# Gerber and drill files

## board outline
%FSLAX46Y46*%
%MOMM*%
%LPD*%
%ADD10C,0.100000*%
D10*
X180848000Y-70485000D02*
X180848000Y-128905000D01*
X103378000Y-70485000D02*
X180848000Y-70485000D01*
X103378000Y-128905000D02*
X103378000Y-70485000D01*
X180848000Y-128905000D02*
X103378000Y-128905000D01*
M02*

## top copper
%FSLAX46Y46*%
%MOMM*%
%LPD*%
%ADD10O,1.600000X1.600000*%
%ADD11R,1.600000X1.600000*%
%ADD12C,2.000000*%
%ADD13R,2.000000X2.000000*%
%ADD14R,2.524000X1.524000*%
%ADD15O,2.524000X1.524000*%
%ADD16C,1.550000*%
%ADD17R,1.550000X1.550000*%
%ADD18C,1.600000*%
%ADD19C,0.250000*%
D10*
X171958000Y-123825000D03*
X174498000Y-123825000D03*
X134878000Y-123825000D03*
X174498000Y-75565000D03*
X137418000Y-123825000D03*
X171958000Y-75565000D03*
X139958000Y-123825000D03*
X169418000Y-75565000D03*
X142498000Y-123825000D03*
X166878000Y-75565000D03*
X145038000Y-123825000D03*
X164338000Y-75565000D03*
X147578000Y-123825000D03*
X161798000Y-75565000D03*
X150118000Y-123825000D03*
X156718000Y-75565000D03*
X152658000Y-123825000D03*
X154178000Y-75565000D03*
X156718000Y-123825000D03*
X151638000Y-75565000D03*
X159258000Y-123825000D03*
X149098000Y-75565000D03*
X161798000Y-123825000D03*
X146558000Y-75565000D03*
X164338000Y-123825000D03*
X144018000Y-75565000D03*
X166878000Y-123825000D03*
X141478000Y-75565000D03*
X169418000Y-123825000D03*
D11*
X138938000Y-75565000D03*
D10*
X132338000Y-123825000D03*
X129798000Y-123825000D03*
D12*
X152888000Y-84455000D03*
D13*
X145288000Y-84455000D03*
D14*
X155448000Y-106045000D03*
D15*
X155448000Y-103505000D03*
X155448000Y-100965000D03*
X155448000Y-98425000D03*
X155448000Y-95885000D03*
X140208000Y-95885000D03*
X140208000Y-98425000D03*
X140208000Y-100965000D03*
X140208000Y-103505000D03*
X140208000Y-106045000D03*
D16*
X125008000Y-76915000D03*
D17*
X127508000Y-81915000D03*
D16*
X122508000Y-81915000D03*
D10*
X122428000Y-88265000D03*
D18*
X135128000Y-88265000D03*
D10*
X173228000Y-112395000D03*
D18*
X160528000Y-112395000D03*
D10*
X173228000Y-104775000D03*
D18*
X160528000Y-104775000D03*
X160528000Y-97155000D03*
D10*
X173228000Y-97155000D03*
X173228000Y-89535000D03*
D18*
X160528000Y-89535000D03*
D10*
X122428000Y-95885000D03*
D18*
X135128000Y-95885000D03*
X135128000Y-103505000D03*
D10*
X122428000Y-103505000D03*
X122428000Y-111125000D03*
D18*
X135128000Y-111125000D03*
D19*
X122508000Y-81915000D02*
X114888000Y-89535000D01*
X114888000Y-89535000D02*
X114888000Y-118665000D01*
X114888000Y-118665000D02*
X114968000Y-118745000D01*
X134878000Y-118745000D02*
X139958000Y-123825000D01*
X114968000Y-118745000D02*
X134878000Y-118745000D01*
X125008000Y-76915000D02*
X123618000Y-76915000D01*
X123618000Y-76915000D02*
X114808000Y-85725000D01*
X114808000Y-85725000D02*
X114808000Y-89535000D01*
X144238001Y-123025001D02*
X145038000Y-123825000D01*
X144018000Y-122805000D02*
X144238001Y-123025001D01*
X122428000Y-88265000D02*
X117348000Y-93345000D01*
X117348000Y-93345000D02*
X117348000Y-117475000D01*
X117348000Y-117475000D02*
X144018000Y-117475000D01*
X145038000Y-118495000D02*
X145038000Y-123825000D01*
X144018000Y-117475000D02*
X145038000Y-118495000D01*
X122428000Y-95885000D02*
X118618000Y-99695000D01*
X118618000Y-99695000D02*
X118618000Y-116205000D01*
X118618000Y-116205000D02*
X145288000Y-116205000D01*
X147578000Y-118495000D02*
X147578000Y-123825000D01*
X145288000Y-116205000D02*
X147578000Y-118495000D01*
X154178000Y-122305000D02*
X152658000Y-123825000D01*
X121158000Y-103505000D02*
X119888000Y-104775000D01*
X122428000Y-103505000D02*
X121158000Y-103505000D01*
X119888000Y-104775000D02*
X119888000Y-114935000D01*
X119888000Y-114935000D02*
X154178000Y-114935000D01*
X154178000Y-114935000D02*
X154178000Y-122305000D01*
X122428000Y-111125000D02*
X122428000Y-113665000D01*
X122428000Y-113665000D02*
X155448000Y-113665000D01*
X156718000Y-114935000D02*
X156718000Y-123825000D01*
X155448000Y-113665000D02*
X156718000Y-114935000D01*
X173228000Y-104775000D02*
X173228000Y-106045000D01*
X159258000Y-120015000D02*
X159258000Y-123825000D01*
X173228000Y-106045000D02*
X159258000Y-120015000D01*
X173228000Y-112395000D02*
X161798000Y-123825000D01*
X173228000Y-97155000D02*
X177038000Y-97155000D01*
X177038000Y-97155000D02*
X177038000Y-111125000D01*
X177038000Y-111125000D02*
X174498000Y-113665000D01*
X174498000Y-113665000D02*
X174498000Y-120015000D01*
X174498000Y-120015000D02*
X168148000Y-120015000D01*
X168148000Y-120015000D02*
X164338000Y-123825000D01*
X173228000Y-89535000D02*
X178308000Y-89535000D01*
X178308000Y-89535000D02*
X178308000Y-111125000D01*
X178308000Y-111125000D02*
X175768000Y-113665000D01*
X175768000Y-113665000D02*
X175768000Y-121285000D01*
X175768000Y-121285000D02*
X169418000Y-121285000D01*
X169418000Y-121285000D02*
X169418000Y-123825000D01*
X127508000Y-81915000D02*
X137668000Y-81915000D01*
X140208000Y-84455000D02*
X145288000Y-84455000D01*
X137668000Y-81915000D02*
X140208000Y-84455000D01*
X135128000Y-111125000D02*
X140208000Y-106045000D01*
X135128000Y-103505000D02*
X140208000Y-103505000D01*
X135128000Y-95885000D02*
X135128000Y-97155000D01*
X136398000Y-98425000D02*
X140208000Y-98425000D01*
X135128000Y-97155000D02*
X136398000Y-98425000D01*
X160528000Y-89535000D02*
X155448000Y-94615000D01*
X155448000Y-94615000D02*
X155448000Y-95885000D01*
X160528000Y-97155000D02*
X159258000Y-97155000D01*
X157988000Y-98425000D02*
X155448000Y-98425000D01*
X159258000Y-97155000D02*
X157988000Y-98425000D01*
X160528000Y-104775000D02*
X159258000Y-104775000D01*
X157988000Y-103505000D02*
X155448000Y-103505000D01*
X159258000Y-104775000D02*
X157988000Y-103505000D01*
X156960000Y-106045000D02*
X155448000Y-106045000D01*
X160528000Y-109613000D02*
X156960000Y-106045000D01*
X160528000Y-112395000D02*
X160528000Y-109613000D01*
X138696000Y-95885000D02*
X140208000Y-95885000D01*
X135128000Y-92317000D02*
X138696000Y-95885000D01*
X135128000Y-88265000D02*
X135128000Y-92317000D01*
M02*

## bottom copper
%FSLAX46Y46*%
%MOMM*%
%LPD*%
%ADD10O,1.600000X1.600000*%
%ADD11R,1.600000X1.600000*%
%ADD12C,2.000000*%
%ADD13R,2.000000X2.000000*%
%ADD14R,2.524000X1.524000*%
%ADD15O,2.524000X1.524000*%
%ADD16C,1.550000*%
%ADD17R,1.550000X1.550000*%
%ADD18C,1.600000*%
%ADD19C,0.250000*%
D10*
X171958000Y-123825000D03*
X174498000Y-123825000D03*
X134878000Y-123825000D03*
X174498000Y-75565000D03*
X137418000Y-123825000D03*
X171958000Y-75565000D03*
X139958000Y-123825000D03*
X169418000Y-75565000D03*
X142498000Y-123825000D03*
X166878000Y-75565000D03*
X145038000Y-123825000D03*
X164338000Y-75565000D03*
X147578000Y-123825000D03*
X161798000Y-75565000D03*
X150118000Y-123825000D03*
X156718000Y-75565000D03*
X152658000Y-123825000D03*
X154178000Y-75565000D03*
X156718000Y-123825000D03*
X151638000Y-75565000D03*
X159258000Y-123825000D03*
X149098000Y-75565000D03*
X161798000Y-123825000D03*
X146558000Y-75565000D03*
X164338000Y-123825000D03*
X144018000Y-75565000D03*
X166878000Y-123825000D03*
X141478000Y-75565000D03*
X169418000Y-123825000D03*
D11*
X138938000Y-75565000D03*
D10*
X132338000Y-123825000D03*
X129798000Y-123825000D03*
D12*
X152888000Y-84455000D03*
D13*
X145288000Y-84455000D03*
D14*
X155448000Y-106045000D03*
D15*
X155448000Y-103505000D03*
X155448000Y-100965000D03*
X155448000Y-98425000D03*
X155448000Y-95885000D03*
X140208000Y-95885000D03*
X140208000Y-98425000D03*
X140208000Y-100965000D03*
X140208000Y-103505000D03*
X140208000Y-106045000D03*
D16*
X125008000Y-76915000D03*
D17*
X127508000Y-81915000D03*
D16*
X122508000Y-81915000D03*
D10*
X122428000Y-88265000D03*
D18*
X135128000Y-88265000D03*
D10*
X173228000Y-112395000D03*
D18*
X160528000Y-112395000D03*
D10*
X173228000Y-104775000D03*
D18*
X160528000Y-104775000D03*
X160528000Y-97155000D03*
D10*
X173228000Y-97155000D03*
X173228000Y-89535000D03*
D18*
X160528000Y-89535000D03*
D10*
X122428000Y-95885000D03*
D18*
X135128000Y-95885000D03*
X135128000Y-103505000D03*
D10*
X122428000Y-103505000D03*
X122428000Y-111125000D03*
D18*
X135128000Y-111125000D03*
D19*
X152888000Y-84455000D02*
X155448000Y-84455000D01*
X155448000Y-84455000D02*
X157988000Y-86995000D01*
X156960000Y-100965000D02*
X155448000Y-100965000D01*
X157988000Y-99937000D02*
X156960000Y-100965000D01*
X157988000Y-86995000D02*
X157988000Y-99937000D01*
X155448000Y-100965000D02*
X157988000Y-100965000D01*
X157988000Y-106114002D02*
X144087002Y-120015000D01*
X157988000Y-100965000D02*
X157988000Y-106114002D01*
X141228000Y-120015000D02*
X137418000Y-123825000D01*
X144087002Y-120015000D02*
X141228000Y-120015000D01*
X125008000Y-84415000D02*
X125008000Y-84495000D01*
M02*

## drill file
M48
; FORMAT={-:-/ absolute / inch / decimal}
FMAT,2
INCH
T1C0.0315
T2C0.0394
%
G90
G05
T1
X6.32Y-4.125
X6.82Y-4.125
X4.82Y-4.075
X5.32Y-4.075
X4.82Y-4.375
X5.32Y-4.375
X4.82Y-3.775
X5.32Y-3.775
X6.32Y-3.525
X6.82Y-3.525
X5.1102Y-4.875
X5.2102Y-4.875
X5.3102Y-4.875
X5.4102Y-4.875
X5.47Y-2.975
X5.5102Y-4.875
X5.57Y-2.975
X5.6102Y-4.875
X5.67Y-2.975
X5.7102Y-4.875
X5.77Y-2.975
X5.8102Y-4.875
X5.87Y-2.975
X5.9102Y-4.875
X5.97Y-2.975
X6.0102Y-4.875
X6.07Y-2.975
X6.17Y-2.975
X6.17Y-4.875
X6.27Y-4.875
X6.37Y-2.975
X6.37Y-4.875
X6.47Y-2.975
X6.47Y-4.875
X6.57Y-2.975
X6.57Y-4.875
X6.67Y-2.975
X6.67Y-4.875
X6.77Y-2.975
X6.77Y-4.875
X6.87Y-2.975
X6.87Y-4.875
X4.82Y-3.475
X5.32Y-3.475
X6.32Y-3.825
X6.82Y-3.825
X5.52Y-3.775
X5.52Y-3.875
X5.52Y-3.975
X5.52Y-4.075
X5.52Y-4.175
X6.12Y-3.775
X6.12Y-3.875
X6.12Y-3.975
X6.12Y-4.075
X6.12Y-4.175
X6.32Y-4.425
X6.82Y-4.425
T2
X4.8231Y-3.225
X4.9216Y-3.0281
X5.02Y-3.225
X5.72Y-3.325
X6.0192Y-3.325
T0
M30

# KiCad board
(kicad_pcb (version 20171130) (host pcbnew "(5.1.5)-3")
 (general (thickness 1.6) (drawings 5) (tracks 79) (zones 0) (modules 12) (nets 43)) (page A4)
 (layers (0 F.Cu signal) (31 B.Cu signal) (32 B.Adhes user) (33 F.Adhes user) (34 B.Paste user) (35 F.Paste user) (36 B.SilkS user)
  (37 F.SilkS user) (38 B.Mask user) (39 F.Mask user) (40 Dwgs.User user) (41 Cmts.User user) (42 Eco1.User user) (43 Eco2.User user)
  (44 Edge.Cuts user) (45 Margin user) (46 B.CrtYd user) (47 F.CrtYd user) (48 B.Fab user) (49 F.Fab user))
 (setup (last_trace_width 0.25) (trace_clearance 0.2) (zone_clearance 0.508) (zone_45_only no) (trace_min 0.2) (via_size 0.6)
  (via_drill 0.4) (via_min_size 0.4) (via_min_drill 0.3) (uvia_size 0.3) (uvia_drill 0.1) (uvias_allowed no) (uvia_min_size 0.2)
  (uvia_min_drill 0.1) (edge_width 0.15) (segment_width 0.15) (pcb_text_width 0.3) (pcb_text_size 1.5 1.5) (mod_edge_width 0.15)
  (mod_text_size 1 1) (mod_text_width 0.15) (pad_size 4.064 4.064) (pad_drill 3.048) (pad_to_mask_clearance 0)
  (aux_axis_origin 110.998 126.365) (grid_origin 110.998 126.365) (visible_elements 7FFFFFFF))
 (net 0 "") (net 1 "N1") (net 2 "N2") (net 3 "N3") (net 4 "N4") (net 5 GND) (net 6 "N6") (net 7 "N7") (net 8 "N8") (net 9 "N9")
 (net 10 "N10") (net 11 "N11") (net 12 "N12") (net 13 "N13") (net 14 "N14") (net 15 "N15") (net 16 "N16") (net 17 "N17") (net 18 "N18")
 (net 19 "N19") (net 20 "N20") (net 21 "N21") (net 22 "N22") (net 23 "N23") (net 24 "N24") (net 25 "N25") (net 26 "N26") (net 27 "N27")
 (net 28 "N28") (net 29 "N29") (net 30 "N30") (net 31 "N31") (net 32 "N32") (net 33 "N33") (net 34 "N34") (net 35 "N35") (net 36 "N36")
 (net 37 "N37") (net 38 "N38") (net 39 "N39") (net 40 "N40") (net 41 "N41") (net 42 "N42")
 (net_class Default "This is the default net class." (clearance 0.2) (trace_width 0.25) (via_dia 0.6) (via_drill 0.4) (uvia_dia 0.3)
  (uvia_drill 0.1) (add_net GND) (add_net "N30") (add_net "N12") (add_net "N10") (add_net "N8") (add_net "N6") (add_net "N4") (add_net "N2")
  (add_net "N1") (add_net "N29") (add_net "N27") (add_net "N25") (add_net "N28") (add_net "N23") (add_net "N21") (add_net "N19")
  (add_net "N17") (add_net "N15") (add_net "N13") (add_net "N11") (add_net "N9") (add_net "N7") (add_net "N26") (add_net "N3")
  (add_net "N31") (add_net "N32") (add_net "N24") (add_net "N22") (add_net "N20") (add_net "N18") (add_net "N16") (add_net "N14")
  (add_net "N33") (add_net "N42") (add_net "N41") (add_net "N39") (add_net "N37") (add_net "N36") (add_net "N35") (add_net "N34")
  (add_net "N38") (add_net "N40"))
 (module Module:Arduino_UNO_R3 (layer F.Cu) (at 138.938 75.565)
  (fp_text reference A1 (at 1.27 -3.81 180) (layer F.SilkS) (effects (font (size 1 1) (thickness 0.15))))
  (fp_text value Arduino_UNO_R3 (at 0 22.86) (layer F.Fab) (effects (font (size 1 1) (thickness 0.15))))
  (pad 16 thru_hole oval (at 33.02 48.26 90) (size 1.6 1.6) (drill 0.8) (layers *.Cu *.Mask) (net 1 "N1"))
  (pad 15 thru_hole oval (at 35.56 48.26 90) (size 1.6 1.6) (drill 0.8) (layers *.Cu *.Mask) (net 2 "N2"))
  (pad 30 thru_hole oval (at -4.06 48.26 90) (size 1.6 1.6) (drill 0.8) (layers *.Cu *.Mask) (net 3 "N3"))
  (pad 14 thru_hole oval (at 35.56 0 90) (size 1.6 1.6) (drill 0.8) (layers *.Cu *.Mask) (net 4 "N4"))
  (pad 29 thru_hole oval (at -1.52 48.26 90) (size 1.6 1.6) (drill 0.8) (layers *.Cu *.Mask) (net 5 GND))
  (pad 13 thru_hole oval (at 33.02 0 90) (size 1.6 1.6) (drill 0.8) (layers *.Cu *.Mask) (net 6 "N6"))
  (pad 28 thru_hole oval (at 1.02 48.26 90) (size 1.6 1.6) (drill 0.8) (layers *.Cu *.Mask) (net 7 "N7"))
  (pad 12 thru_hole oval (at 30.48 0 90) (size 1.6 1.6) (drill 0.8) (layers *.Cu *.Mask) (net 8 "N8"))
  (pad 27 thru_hole oval (at 3.56 48.26 90) (size 1.6 1.6) (drill 0.8) (layers *.Cu *.Mask) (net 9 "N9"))
  (pad 11 thru_hole oval (at 27.94 0 90) (size 1.6 1.6) (drill 0.8) (layers *.Cu *.Mask) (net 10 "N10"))
  (pad 26 thru_hole oval (at 6.1 48.26 90) (size 1.6 1.6) (drill 0.8) (layers *.Cu *.Mask) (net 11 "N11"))
  (pad 10 thru_hole oval (at 25.4 0 90) (size 1.6 1.6) (drill 0.8) (layers *.Cu *.Mask) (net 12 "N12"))
  (pad 25 thru_hole oval (at 8.64 48.26 90) (size 1.6 1.6) (drill 0.8) (layers *.Cu *.Mask) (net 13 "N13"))
  (pad 9 thru_hole oval (at 22.86 0 90) (size 1.6 1.6) (drill 0.8) (layers *.Cu *.Mask) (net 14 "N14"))
  (pad 24 thru_hole oval (at 11.18 48.26 90) (size 1.6 1.6) (drill 0.8) (layers *.Cu *.Mask) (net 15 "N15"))
  (pad 8 thru_hole oval (at 17.78 0 90) (size 1.6 1.6) (drill 0.8) (layers *.Cu *.Mask) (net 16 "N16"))
  (pad 23 thru_hole oval (at 13.72 48.26 90) (size 1.6 1.6) (drill 0.8) (layers *.Cu *.Mask) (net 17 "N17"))
  (pad 7 thru_hole oval (at 15.24 0 90) (size 1.6 1.6) (drill 0.8) (layers *.Cu *.Mask) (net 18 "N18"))
  (pad 22 thru_hole oval (at 17.78 48.26 90) (size 1.6 1.6) (drill 0.8) (layers *.Cu *.Mask) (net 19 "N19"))
  (pad 6 thru_hole oval (at 12.7 0 90) (size 1.6 1.6) (drill 0.8) (layers *.Cu *.Mask) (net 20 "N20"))
  (pad 21 thru_hole oval (at 20.32 48.26 90) (size 1.6 1.6) (drill 0.8) (layers *.Cu *.Mask) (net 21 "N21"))
  (pad 5 thru_hole oval (at 10.16 0 90) (size 1.6 1.6) (drill 0.8) (layers *.Cu *.Mask) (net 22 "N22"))
  (pad 20 thru_hole oval (at 22.86 48.26 90) (size 1.6 1.6) (drill 0.8) (layers *.Cu *.Mask) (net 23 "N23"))
  (pad 4 thru_hole oval (at 7.62 0 90) (size 1.6 1.6) (drill 0.8) (layers *.Cu *.Mask) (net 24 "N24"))
  (pad 19 thru_hole oval (at 25.4 48.26 90) (size 1.6 1.6) (drill 0.8) (layers *.Cu *.Mask) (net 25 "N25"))
  (pad 3 thru_hole oval (at 5.08 0 90) (size 1.6 1.6) (drill 0.8) (layers *.Cu *.Mask) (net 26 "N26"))
  (pad 18 thru_hole oval (at 27.94 48.26 90) (size 1.6 1.6) (drill 0.8) (layers *.Cu *.Mask) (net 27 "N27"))
  (pad 2 thru_hole oval (at 2.54 0 90) (size 1.6 1.6) (drill 0.8) (layers *.Cu *.Mask) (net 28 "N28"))
  (pad 17 thru_hole oval (at 30.48 48.26 90) (size 1.6 1.6) (drill 0.8) (layers *.Cu *.Mask) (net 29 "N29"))
  (pad 1 thru_hole rect (at 0 0 90) (size 1.6 1.6) (drill 0.8) (layers *.Cu *.Mask) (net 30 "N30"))
  (pad 31 thru_hole oval (at -6.6 48.26 90) (size 1.6 1.6) (drill 0.8) (layers *.Cu *.Mask) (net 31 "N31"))
  (pad 32 thru_hole oval (at -9.14 48.26 90) (size 1.6 1.6) (drill 0.8) (layers *.Cu *.Mask) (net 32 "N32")))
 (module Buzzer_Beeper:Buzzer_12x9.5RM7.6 (layer F.Cu) (at 145.288 84.455)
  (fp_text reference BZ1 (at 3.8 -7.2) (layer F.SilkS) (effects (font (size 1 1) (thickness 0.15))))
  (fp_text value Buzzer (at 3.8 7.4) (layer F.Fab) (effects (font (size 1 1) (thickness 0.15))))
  (pad 2 thru_hole circle (at 7.6 0) (size 2 2) (drill 1) (layers *.Cu *.Mask) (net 5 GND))
  (pad 1 thru_hole rect (at 0 0) (size 2 2) (drill 1) (layers *.Cu *.Mask) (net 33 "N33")))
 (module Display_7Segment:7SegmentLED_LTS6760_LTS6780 (layer F.Cu) (at 155.448 106.045 180)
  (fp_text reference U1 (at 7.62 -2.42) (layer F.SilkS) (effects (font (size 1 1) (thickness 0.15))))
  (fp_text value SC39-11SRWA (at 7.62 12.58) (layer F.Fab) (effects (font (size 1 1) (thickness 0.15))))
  (pad 1 thru_hole rect (at 0 0 90) (size 1.524 2.524) (drill 0.8) (layers *.Cu *.Mask) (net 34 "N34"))
  (pad 2 thru_hole oval (at 0 2.54 90) (size 1.524 2.524) (drill 0.8) (layers *.Cu *.Mask) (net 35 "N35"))
  (pad 3 thru_hole oval (at 0 5.08 90) (size 1.524 2.524) (drill 0.8) (layers *.Cu *.Mask) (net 5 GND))
  (pad 4 thru_hole oval (at 0 7.62 90) (size 1.524 2.524) (drill 0.8) (layers *.Cu *.Mask) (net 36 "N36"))
  (pad 5 thru_hole oval (at 0 10.16 90) (size 1.524 2.524) (drill 0.8) (layers *.Cu *.Mask) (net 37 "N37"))
  (pad 6 thru_hole oval (at 15.24 10.16 90) (size 1.524 2.524) (drill 0.8) (layers *.Cu *.Mask) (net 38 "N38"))
  (pad 7 thru_hole oval (at 15.24 7.62 90) (size 1.524 2.524) (drill 0.8) (layers *.Cu *.Mask) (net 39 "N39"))
  (pad 8 thru_hole oval (at 15.24 5.08 90) (size 1.524 2.524) (drill 0.8) (layers *.Cu *.Mask) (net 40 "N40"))
  (pad 9 thru_hole oval (at 15.24 2.54 90) (size 1.524 2.524) (drill 0.8) (layers *.Cu *.Mask) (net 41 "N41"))
  (pad 10 thru_hole oval (at 15.24 0 90) (size 1.524 2.524) (drill 0.8) (layers *.Cu *.Mask) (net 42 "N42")))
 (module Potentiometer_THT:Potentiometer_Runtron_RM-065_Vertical (layer F.Cu) (at 127.508 81.915 180)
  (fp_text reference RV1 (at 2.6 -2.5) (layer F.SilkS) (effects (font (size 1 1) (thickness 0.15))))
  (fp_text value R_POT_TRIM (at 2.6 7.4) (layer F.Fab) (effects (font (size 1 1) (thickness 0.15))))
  (pad 2 thru_hole circle (at 2.5 5 180) (size 1.55 1.55) (drill 1) (layers *.Cu *.Mask) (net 7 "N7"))
  (pad 1 thru_hole rect (at 0 0 180) (size 1.55 1.55) (drill 1) (layers *.Cu *.Mask) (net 33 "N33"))
  (pad 3 thru_hole circle (at 5 0 180) (size 1.55 1.55) (drill 1) (layers *.Cu *.Mask) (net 7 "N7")))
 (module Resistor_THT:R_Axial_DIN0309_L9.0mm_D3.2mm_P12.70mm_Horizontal (layer F.Cu) (at 135.128 88.265 180)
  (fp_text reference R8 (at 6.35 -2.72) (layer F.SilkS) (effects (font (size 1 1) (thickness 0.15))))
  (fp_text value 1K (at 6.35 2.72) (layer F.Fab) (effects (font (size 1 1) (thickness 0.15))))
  (pad 2 thru_hole oval (at 12.7 0 180) (size 1.6 1.6) (drill 0.8) (layers *.Cu *.Mask) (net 11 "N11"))
  (pad 1 thru_hole circle (at 0 0 180) (size 1.6 1.6) (drill 0.8) (layers *.Cu *.Mask) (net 38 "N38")))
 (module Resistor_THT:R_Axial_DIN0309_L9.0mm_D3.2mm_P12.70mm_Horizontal (layer F.Cu) (at 160.528 112.395)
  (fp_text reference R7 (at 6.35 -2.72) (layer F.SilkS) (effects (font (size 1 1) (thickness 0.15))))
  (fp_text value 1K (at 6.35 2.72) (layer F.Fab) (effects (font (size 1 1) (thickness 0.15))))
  (pad 2 thru_hole oval (at 12.7 0) (size 1.6 1.6) (drill 0.8) (layers *.Cu *.Mask) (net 23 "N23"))
  (pad 1 thru_hole circle (at 0 0) (size 1.6 1.6) (drill 0.8) (layers *.Cu *.Mask) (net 34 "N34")))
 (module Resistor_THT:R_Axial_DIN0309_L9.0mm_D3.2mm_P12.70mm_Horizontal (layer F.Cu) (at 160.528 104.775)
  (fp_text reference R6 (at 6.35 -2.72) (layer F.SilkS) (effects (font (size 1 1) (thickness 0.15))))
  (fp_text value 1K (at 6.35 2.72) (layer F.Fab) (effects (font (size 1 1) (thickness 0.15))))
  (pad 2 thru_hole oval (at 12.7 0) (size 1.6 1.6) (drill 0.8) (layers *.Cu *.Mask) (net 21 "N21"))
  (pad 1 thru_hole circle (at 0 0) (size 1.6 1.6) (drill 0.8) (layers *.Cu *.Mask) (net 35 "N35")))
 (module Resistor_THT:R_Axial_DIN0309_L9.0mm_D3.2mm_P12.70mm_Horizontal (layer F.Cu) (at 160.528 97.155)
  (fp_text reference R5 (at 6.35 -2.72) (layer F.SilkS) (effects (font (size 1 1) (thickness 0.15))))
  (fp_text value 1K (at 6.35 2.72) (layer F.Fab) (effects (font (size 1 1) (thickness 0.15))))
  (pad 1 thru_hole circle (at 0 0) (size 1.6 1.6) (drill 0.8) (layers *.Cu *.Mask) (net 36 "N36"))
  (pad 2 thru_hole oval (at 12.7 0) (size 1.6 1.6) (drill 0.8) (layers *.Cu *.Mask) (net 25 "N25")))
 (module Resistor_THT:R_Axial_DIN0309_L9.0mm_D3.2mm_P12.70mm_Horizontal (layer F.Cu) (at 160.528 89.535)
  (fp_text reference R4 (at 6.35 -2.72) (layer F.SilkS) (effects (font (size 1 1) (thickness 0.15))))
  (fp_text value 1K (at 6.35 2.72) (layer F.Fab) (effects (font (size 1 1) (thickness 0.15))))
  (pad 2 thru_hole oval (at 12.7 0) (size 1.6 1.6) (drill 0.8) (layers *.Cu *.Mask) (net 29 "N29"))
  (pad 1 thru_hole circle (at 0 0) (size 1.6 1.6) (drill 0.8) (layers *.Cu *.Mask) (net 37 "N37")))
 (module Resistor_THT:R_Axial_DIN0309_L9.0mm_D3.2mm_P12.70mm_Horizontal (layer F.Cu) (at 135.128 95.885 180)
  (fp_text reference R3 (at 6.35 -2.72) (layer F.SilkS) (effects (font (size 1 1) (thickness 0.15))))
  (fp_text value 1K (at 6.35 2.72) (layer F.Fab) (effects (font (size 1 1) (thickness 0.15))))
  (pad 2 thru_hole oval (at 12.7 0 180) (size 1.6 1.6) (drill 0.8) (layers *.Cu *.Mask) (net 13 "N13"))
  (pad 1 thru_hole circle (at 0 0 180) (size 1.6 1.6) (drill 0.8) (layers *.Cu *.Mask) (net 39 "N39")))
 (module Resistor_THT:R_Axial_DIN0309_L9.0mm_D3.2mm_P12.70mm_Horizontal (layer F.Cu) (at 135.128 103.505 180)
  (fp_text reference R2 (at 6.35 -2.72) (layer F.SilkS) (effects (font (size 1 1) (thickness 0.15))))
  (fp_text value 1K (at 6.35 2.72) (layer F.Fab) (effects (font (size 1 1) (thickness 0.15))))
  (pad 1 thru_hole circle (at 0 0 180) (size 1.6 1.6) (drill 0.8) (layers *.Cu *.Mask) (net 41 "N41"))
  (pad 2 thru_hole oval (at 12.7 0 180) (size 1.6 1.6) (drill 0.8) (layers *.Cu *.Mask) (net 17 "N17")))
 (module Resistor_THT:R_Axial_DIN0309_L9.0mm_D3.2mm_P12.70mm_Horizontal (layer F.Cu) (at 135.128 111.125 180)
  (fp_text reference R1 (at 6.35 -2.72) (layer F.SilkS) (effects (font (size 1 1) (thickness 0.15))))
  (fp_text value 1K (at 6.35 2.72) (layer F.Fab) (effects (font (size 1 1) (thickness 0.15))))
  (pad 2 thru_hole oval (at 12.7 0 180) (size 1.6 1.6) (drill 0.8) (layers *.Cu *.Mask) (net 19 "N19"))
  (pad 1 thru_hole circle (at 0 0 180) (size 1.6 1.6) (drill 0.8) (layers *.Cu *.Mask) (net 42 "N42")))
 (gr_line (start 180.848 70.485) (end 180.848 128.905) (layer Edge.Cuts) (width 0.1))
 (gr_line (start 103.378 70.485) (end 180.848 70.485) (layer Edge.Cuts) (width 0.1))
 (gr_line (start 103.378 128.905) (end 103.378 70.485) (layer Edge.Cuts) (width 0.1))
 (gr_line (start 180.848 128.905) (end 103.378 128.905) (layer Edge.Cuts) (width 0.1))
 (segment (start 152.888 84.455) (end 155.448 84.455) (width 0.25) (layer B.Cu) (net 5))
 (segment (start 155.448 84.455) (end 157.988 86.995) (width 0.25) (layer B.Cu) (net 5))
 (segment (start 156.96 100.965) (end 155.448 100.965) (width 0.25) (layer B.Cu) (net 5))
 (segment (start 157.988 99.937) (end 156.96 100.965) (width 0.25) (layer B.Cu) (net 5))
 (segment (start 157.988 86.995) (end 157.988 99.937) (width 0.25) (layer B.Cu) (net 5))
 (segment (start 155.448 100.965) (end 157.988 100.965) (width 0.25) (layer B.Cu) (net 5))
 (segment (start 157.988 106.114002) (end 144.087002 120.015) (width 0.25) (layer B.Cu) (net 5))
 (segment (start 157.988 100.965) (end 157.988 106.114002) (width 0.25) (layer B.Cu) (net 5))
 (segment (start 141.228 120.015) (end 137.418 123.825) (width 0.25) (layer B.Cu) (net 5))
 (segment (start 144.087002 120.015) (end 141.228 120.015) (width 0.25) (layer B.Cu) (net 5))
 (segment (start 125.008 84.415) (end 125.008 84.495) (width 0.25) (layer B.Cu) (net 7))
 (segment (start 122.508 81.915) (end 114.888 89.535) (width 0.25) (layer F.Cu) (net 7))
 (segment (start 114.888 89.535) (end 114.888 118.665) (width 0.25) (layer F.Cu) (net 7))
 (segment (start 114.888 118.665) (end 114.968 118.745) (width 0.25) (layer F.Cu) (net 7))
 (segment (start 134.878 118.745) (end 139.958 123.825) (width 0.25) (layer F.Cu) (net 7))
 (segment (start 114.968 118.745) (end 134.878 118.745) (width 0.25) (layer F.Cu) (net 7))
 (segment (start 125.008 76.915) (end 123.618 76.915) (width 0.25) (layer F.Cu) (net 7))
 (segment (start 123.618 76.915) (end 114.808 85.725) (width 0.25) (layer F.Cu) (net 7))
 (segment (start 114.808 85.725) (end 114.808 89.535) (width 0.25) (layer F.Cu) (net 7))
 (segment (start 144.238001 123.025001) (end 145.038 123.825) (width 0.25) (layer F.Cu) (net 11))
 (segment (start 144.018 122.805) (end 144.238001 123.025001) (width 0.25) (layer F.Cu) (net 11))
 (segment (start 122.428 88.265) (end 117.348 93.345) (width 0.25) (layer F.Cu) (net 11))
 (segment (start 117.348 93.345) (end 117.348 117.475) (width 0.25) (layer F.Cu) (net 11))
 (segment (start 117.348 117.475) (end 144.018 117.475) (width 0.25) (layer F.Cu) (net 11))
 (segment (start 145.038 118.495) (end 145.038 123.825) (width 0.25) (layer F.Cu) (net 11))
 (segment (start 144.018 117.475) (end 145.038 118.495) (width 0.25) (layer F.Cu) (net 11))
 (segment (start 122.428 95.885) (end 118.618 99.695) (width 0.25) (layer F.Cu) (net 13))
 (segment (start 118.618 99.695) (end 118.618 116.205) (width 0.25) (layer F.Cu) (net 13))
 (segment (start 118.618 116.205) (end 145.288 116.205) (width 0.25) (layer F.Cu) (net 13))
 (segment (start 147.578 118.495) (end 147.578 123.825) (width 0.25) (layer F.Cu) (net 13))
 (segment (start 145.288 116.205) (end 147.578 118.495) (width 0.25) (layer F.Cu) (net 13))
 (segment (start 154.178 122.305) (end 152.658 123.825) (width 0.25) (layer F.Cu) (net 17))
 (segment (start 121.158 103.505) (end 119.888 104.775) (width 0.25) (layer F.Cu) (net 17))
 (segment (start 122.428 103.505) (end 121.158 103.505) (width 0.25) (layer F.Cu) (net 17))
 (segment (start 119.888 104.775) (end 119.888 114.935) (width 0.25) (layer F.Cu) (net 17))
 (segment (start 119.888 114.935) (end 154.178 114.935) (width 0.25) (layer F.Cu) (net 17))
 (segment (start 154.178 114.935) (end 154.178 122.305) (width 0.25) (layer F.Cu) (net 17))
 (segment (start 122.428 111.125) (end 122.428 113.665) (width 0.25) (layer F.Cu) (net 19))
 (segment (start 122.428 113.665) (end 155.448 113.665) (width 0.25) (layer F.Cu) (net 19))
 (segment (start 156.718 114.935) (end 156.718 123.825) (width 0.25) (layer F.Cu) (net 19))
 (segment (start 155.448 113.665) (end 156.718 114.935) (width 0.25) (layer F.Cu) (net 19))
 (segment (start 173.228 104.775) (end 173.228 106.045) (width 0.25) (layer F.Cu) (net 21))
 (segment (start 159.258 120.015) (end 159.258 123.825) (width 0.25) (layer F.Cu) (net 21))
 (segment (start 173.228 106.045) (end 159.258 120.015) (width 0.25) (layer F.Cu) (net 21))
 (segment (start 173.228 112.395) (end 161.798 123.825) (width 0.25) (layer F.Cu) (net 23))
 (segment (start 173.228 97.155) (end 177.038 97.155) (width 0.25) (layer F.Cu) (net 25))
 (segment (start 177.038 97.155) (end 177.038 111.125) (width 0.25) (layer F.Cu) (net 25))
 (segment (start 177.038 111.125) (end 174.498 113.665) (width 0.25) (layer F.Cu) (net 25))
 (segment (start 174.498 113.665) (end 174.498 120.015) (width 0.25) (layer F.Cu) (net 25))
 (segment (start 174.498 120.015) (end 168.148 120.015) (width 0.25) (layer F.Cu) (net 25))
 (segment (start 168.148 120.015) (end 164.338 123.825) (width 0.25) (layer F.Cu) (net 25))
 (segment (start 173.228 89.535) (end 178.308 89.535) (width 0.25) (layer F.Cu) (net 29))
 (segment (start 178.308 89.535) (end 178.308 111.125) (width 0.25) (layer F.Cu) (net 29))
 (segment (start 178.308 111.125) (end 175.768 113.665) (width 0.25) (layer F.Cu) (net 29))
 (segment (start 175.768 113.665) (end 175.768 121.285) (width 0.25) (layer F.Cu) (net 29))
 (segment (start 175.768 121.285) (end 169.418 121.285) (width 0.25) (layer F.Cu) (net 29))
 (segment (start 169.418 121.285) (end 169.418 123.825) (width 0.25) (layer F.Cu) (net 29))
 (segment (start 127.508 81.915) (end 137.668 81.915) (width 0.25) (layer F.Cu) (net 33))
 (segment (start 140.208 84.455) (end 145.288 84.455) (width 0.25) (layer F.Cu) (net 33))
 (segment (start 137.668 81.915) (end 140.208 84.455) (width 0.25) (layer F.Cu) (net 33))
 (segment (start 135.128 111.125) (end 140.208 106.045) (width 0.25) (layer F.Cu) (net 42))
 (segment (start 135.128 103.505) (end 140.208 103.505) (width 0.25) (layer F.Cu) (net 41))
 (segment (start 135.128 95.885) (end 135.128 97.155) (width 0.25) (layer F.Cu) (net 39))
 (segment (start 136.398 98.425) (end 140.208 98.425) (width 0.25) (layer F.Cu) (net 39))
 (segment (start 135.128 97.155) (end 136.398 98.425) (width 0.25) (layer F.Cu) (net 39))
 (segment (start 160.528 89.535) (end 155.448 94.615) (width 0.25) (layer F.Cu) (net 37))
 (segment (start 155.448 94.615) (end 155.448 95.885) (width 0.25) (layer F.Cu) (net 37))
 (segment (start 160.528 97.155) (end 159.258 97.155) (width 0.25) (layer F.Cu) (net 36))
 (segment (start 157.988 98.425) (end 155.448 98.425) (width 0.25) (layer F.Cu) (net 36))
 (segment (start 159.258 97.155) (end 157.988 98.425) (width 0.25) (layer F.Cu) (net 36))
 (segment (start 160.528 104.775) (end 159.258 104.775) (width 0.25) (layer F.Cu) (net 35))
 (segment (start 157.988 103.505) (end 155.448 103.505) (width 0.25) (layer F.Cu) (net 35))
 (segment (start 159.258 104.775) (end 157.988 103.505) (width 0.25) (layer F.Cu) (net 35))
 (segment (start 156.96 106.045) (end 155.448 106.045) (width 0.25) (layer F.Cu) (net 34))
 (segment (start 160.528 109.613) (end 156.96 106.045) (width 0.25) (layer F.Cu) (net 34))
 (segment (start 160.528 112.395) (end 160.528 109.613) (width 0.25) (layer F.Cu) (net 34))
 (segment (start 138.696 95.885) (end 140.208 95.885) (width 0.25) (layer F.Cu) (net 38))
 (segment (start 135.128 92.317) (end 138.696 95.885) (width 0.25) (layer F.Cu) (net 38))
 (segment (start 135.128 88.265) (end 135.128 92.317) (width 0.25) (layer F.Cu) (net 38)))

